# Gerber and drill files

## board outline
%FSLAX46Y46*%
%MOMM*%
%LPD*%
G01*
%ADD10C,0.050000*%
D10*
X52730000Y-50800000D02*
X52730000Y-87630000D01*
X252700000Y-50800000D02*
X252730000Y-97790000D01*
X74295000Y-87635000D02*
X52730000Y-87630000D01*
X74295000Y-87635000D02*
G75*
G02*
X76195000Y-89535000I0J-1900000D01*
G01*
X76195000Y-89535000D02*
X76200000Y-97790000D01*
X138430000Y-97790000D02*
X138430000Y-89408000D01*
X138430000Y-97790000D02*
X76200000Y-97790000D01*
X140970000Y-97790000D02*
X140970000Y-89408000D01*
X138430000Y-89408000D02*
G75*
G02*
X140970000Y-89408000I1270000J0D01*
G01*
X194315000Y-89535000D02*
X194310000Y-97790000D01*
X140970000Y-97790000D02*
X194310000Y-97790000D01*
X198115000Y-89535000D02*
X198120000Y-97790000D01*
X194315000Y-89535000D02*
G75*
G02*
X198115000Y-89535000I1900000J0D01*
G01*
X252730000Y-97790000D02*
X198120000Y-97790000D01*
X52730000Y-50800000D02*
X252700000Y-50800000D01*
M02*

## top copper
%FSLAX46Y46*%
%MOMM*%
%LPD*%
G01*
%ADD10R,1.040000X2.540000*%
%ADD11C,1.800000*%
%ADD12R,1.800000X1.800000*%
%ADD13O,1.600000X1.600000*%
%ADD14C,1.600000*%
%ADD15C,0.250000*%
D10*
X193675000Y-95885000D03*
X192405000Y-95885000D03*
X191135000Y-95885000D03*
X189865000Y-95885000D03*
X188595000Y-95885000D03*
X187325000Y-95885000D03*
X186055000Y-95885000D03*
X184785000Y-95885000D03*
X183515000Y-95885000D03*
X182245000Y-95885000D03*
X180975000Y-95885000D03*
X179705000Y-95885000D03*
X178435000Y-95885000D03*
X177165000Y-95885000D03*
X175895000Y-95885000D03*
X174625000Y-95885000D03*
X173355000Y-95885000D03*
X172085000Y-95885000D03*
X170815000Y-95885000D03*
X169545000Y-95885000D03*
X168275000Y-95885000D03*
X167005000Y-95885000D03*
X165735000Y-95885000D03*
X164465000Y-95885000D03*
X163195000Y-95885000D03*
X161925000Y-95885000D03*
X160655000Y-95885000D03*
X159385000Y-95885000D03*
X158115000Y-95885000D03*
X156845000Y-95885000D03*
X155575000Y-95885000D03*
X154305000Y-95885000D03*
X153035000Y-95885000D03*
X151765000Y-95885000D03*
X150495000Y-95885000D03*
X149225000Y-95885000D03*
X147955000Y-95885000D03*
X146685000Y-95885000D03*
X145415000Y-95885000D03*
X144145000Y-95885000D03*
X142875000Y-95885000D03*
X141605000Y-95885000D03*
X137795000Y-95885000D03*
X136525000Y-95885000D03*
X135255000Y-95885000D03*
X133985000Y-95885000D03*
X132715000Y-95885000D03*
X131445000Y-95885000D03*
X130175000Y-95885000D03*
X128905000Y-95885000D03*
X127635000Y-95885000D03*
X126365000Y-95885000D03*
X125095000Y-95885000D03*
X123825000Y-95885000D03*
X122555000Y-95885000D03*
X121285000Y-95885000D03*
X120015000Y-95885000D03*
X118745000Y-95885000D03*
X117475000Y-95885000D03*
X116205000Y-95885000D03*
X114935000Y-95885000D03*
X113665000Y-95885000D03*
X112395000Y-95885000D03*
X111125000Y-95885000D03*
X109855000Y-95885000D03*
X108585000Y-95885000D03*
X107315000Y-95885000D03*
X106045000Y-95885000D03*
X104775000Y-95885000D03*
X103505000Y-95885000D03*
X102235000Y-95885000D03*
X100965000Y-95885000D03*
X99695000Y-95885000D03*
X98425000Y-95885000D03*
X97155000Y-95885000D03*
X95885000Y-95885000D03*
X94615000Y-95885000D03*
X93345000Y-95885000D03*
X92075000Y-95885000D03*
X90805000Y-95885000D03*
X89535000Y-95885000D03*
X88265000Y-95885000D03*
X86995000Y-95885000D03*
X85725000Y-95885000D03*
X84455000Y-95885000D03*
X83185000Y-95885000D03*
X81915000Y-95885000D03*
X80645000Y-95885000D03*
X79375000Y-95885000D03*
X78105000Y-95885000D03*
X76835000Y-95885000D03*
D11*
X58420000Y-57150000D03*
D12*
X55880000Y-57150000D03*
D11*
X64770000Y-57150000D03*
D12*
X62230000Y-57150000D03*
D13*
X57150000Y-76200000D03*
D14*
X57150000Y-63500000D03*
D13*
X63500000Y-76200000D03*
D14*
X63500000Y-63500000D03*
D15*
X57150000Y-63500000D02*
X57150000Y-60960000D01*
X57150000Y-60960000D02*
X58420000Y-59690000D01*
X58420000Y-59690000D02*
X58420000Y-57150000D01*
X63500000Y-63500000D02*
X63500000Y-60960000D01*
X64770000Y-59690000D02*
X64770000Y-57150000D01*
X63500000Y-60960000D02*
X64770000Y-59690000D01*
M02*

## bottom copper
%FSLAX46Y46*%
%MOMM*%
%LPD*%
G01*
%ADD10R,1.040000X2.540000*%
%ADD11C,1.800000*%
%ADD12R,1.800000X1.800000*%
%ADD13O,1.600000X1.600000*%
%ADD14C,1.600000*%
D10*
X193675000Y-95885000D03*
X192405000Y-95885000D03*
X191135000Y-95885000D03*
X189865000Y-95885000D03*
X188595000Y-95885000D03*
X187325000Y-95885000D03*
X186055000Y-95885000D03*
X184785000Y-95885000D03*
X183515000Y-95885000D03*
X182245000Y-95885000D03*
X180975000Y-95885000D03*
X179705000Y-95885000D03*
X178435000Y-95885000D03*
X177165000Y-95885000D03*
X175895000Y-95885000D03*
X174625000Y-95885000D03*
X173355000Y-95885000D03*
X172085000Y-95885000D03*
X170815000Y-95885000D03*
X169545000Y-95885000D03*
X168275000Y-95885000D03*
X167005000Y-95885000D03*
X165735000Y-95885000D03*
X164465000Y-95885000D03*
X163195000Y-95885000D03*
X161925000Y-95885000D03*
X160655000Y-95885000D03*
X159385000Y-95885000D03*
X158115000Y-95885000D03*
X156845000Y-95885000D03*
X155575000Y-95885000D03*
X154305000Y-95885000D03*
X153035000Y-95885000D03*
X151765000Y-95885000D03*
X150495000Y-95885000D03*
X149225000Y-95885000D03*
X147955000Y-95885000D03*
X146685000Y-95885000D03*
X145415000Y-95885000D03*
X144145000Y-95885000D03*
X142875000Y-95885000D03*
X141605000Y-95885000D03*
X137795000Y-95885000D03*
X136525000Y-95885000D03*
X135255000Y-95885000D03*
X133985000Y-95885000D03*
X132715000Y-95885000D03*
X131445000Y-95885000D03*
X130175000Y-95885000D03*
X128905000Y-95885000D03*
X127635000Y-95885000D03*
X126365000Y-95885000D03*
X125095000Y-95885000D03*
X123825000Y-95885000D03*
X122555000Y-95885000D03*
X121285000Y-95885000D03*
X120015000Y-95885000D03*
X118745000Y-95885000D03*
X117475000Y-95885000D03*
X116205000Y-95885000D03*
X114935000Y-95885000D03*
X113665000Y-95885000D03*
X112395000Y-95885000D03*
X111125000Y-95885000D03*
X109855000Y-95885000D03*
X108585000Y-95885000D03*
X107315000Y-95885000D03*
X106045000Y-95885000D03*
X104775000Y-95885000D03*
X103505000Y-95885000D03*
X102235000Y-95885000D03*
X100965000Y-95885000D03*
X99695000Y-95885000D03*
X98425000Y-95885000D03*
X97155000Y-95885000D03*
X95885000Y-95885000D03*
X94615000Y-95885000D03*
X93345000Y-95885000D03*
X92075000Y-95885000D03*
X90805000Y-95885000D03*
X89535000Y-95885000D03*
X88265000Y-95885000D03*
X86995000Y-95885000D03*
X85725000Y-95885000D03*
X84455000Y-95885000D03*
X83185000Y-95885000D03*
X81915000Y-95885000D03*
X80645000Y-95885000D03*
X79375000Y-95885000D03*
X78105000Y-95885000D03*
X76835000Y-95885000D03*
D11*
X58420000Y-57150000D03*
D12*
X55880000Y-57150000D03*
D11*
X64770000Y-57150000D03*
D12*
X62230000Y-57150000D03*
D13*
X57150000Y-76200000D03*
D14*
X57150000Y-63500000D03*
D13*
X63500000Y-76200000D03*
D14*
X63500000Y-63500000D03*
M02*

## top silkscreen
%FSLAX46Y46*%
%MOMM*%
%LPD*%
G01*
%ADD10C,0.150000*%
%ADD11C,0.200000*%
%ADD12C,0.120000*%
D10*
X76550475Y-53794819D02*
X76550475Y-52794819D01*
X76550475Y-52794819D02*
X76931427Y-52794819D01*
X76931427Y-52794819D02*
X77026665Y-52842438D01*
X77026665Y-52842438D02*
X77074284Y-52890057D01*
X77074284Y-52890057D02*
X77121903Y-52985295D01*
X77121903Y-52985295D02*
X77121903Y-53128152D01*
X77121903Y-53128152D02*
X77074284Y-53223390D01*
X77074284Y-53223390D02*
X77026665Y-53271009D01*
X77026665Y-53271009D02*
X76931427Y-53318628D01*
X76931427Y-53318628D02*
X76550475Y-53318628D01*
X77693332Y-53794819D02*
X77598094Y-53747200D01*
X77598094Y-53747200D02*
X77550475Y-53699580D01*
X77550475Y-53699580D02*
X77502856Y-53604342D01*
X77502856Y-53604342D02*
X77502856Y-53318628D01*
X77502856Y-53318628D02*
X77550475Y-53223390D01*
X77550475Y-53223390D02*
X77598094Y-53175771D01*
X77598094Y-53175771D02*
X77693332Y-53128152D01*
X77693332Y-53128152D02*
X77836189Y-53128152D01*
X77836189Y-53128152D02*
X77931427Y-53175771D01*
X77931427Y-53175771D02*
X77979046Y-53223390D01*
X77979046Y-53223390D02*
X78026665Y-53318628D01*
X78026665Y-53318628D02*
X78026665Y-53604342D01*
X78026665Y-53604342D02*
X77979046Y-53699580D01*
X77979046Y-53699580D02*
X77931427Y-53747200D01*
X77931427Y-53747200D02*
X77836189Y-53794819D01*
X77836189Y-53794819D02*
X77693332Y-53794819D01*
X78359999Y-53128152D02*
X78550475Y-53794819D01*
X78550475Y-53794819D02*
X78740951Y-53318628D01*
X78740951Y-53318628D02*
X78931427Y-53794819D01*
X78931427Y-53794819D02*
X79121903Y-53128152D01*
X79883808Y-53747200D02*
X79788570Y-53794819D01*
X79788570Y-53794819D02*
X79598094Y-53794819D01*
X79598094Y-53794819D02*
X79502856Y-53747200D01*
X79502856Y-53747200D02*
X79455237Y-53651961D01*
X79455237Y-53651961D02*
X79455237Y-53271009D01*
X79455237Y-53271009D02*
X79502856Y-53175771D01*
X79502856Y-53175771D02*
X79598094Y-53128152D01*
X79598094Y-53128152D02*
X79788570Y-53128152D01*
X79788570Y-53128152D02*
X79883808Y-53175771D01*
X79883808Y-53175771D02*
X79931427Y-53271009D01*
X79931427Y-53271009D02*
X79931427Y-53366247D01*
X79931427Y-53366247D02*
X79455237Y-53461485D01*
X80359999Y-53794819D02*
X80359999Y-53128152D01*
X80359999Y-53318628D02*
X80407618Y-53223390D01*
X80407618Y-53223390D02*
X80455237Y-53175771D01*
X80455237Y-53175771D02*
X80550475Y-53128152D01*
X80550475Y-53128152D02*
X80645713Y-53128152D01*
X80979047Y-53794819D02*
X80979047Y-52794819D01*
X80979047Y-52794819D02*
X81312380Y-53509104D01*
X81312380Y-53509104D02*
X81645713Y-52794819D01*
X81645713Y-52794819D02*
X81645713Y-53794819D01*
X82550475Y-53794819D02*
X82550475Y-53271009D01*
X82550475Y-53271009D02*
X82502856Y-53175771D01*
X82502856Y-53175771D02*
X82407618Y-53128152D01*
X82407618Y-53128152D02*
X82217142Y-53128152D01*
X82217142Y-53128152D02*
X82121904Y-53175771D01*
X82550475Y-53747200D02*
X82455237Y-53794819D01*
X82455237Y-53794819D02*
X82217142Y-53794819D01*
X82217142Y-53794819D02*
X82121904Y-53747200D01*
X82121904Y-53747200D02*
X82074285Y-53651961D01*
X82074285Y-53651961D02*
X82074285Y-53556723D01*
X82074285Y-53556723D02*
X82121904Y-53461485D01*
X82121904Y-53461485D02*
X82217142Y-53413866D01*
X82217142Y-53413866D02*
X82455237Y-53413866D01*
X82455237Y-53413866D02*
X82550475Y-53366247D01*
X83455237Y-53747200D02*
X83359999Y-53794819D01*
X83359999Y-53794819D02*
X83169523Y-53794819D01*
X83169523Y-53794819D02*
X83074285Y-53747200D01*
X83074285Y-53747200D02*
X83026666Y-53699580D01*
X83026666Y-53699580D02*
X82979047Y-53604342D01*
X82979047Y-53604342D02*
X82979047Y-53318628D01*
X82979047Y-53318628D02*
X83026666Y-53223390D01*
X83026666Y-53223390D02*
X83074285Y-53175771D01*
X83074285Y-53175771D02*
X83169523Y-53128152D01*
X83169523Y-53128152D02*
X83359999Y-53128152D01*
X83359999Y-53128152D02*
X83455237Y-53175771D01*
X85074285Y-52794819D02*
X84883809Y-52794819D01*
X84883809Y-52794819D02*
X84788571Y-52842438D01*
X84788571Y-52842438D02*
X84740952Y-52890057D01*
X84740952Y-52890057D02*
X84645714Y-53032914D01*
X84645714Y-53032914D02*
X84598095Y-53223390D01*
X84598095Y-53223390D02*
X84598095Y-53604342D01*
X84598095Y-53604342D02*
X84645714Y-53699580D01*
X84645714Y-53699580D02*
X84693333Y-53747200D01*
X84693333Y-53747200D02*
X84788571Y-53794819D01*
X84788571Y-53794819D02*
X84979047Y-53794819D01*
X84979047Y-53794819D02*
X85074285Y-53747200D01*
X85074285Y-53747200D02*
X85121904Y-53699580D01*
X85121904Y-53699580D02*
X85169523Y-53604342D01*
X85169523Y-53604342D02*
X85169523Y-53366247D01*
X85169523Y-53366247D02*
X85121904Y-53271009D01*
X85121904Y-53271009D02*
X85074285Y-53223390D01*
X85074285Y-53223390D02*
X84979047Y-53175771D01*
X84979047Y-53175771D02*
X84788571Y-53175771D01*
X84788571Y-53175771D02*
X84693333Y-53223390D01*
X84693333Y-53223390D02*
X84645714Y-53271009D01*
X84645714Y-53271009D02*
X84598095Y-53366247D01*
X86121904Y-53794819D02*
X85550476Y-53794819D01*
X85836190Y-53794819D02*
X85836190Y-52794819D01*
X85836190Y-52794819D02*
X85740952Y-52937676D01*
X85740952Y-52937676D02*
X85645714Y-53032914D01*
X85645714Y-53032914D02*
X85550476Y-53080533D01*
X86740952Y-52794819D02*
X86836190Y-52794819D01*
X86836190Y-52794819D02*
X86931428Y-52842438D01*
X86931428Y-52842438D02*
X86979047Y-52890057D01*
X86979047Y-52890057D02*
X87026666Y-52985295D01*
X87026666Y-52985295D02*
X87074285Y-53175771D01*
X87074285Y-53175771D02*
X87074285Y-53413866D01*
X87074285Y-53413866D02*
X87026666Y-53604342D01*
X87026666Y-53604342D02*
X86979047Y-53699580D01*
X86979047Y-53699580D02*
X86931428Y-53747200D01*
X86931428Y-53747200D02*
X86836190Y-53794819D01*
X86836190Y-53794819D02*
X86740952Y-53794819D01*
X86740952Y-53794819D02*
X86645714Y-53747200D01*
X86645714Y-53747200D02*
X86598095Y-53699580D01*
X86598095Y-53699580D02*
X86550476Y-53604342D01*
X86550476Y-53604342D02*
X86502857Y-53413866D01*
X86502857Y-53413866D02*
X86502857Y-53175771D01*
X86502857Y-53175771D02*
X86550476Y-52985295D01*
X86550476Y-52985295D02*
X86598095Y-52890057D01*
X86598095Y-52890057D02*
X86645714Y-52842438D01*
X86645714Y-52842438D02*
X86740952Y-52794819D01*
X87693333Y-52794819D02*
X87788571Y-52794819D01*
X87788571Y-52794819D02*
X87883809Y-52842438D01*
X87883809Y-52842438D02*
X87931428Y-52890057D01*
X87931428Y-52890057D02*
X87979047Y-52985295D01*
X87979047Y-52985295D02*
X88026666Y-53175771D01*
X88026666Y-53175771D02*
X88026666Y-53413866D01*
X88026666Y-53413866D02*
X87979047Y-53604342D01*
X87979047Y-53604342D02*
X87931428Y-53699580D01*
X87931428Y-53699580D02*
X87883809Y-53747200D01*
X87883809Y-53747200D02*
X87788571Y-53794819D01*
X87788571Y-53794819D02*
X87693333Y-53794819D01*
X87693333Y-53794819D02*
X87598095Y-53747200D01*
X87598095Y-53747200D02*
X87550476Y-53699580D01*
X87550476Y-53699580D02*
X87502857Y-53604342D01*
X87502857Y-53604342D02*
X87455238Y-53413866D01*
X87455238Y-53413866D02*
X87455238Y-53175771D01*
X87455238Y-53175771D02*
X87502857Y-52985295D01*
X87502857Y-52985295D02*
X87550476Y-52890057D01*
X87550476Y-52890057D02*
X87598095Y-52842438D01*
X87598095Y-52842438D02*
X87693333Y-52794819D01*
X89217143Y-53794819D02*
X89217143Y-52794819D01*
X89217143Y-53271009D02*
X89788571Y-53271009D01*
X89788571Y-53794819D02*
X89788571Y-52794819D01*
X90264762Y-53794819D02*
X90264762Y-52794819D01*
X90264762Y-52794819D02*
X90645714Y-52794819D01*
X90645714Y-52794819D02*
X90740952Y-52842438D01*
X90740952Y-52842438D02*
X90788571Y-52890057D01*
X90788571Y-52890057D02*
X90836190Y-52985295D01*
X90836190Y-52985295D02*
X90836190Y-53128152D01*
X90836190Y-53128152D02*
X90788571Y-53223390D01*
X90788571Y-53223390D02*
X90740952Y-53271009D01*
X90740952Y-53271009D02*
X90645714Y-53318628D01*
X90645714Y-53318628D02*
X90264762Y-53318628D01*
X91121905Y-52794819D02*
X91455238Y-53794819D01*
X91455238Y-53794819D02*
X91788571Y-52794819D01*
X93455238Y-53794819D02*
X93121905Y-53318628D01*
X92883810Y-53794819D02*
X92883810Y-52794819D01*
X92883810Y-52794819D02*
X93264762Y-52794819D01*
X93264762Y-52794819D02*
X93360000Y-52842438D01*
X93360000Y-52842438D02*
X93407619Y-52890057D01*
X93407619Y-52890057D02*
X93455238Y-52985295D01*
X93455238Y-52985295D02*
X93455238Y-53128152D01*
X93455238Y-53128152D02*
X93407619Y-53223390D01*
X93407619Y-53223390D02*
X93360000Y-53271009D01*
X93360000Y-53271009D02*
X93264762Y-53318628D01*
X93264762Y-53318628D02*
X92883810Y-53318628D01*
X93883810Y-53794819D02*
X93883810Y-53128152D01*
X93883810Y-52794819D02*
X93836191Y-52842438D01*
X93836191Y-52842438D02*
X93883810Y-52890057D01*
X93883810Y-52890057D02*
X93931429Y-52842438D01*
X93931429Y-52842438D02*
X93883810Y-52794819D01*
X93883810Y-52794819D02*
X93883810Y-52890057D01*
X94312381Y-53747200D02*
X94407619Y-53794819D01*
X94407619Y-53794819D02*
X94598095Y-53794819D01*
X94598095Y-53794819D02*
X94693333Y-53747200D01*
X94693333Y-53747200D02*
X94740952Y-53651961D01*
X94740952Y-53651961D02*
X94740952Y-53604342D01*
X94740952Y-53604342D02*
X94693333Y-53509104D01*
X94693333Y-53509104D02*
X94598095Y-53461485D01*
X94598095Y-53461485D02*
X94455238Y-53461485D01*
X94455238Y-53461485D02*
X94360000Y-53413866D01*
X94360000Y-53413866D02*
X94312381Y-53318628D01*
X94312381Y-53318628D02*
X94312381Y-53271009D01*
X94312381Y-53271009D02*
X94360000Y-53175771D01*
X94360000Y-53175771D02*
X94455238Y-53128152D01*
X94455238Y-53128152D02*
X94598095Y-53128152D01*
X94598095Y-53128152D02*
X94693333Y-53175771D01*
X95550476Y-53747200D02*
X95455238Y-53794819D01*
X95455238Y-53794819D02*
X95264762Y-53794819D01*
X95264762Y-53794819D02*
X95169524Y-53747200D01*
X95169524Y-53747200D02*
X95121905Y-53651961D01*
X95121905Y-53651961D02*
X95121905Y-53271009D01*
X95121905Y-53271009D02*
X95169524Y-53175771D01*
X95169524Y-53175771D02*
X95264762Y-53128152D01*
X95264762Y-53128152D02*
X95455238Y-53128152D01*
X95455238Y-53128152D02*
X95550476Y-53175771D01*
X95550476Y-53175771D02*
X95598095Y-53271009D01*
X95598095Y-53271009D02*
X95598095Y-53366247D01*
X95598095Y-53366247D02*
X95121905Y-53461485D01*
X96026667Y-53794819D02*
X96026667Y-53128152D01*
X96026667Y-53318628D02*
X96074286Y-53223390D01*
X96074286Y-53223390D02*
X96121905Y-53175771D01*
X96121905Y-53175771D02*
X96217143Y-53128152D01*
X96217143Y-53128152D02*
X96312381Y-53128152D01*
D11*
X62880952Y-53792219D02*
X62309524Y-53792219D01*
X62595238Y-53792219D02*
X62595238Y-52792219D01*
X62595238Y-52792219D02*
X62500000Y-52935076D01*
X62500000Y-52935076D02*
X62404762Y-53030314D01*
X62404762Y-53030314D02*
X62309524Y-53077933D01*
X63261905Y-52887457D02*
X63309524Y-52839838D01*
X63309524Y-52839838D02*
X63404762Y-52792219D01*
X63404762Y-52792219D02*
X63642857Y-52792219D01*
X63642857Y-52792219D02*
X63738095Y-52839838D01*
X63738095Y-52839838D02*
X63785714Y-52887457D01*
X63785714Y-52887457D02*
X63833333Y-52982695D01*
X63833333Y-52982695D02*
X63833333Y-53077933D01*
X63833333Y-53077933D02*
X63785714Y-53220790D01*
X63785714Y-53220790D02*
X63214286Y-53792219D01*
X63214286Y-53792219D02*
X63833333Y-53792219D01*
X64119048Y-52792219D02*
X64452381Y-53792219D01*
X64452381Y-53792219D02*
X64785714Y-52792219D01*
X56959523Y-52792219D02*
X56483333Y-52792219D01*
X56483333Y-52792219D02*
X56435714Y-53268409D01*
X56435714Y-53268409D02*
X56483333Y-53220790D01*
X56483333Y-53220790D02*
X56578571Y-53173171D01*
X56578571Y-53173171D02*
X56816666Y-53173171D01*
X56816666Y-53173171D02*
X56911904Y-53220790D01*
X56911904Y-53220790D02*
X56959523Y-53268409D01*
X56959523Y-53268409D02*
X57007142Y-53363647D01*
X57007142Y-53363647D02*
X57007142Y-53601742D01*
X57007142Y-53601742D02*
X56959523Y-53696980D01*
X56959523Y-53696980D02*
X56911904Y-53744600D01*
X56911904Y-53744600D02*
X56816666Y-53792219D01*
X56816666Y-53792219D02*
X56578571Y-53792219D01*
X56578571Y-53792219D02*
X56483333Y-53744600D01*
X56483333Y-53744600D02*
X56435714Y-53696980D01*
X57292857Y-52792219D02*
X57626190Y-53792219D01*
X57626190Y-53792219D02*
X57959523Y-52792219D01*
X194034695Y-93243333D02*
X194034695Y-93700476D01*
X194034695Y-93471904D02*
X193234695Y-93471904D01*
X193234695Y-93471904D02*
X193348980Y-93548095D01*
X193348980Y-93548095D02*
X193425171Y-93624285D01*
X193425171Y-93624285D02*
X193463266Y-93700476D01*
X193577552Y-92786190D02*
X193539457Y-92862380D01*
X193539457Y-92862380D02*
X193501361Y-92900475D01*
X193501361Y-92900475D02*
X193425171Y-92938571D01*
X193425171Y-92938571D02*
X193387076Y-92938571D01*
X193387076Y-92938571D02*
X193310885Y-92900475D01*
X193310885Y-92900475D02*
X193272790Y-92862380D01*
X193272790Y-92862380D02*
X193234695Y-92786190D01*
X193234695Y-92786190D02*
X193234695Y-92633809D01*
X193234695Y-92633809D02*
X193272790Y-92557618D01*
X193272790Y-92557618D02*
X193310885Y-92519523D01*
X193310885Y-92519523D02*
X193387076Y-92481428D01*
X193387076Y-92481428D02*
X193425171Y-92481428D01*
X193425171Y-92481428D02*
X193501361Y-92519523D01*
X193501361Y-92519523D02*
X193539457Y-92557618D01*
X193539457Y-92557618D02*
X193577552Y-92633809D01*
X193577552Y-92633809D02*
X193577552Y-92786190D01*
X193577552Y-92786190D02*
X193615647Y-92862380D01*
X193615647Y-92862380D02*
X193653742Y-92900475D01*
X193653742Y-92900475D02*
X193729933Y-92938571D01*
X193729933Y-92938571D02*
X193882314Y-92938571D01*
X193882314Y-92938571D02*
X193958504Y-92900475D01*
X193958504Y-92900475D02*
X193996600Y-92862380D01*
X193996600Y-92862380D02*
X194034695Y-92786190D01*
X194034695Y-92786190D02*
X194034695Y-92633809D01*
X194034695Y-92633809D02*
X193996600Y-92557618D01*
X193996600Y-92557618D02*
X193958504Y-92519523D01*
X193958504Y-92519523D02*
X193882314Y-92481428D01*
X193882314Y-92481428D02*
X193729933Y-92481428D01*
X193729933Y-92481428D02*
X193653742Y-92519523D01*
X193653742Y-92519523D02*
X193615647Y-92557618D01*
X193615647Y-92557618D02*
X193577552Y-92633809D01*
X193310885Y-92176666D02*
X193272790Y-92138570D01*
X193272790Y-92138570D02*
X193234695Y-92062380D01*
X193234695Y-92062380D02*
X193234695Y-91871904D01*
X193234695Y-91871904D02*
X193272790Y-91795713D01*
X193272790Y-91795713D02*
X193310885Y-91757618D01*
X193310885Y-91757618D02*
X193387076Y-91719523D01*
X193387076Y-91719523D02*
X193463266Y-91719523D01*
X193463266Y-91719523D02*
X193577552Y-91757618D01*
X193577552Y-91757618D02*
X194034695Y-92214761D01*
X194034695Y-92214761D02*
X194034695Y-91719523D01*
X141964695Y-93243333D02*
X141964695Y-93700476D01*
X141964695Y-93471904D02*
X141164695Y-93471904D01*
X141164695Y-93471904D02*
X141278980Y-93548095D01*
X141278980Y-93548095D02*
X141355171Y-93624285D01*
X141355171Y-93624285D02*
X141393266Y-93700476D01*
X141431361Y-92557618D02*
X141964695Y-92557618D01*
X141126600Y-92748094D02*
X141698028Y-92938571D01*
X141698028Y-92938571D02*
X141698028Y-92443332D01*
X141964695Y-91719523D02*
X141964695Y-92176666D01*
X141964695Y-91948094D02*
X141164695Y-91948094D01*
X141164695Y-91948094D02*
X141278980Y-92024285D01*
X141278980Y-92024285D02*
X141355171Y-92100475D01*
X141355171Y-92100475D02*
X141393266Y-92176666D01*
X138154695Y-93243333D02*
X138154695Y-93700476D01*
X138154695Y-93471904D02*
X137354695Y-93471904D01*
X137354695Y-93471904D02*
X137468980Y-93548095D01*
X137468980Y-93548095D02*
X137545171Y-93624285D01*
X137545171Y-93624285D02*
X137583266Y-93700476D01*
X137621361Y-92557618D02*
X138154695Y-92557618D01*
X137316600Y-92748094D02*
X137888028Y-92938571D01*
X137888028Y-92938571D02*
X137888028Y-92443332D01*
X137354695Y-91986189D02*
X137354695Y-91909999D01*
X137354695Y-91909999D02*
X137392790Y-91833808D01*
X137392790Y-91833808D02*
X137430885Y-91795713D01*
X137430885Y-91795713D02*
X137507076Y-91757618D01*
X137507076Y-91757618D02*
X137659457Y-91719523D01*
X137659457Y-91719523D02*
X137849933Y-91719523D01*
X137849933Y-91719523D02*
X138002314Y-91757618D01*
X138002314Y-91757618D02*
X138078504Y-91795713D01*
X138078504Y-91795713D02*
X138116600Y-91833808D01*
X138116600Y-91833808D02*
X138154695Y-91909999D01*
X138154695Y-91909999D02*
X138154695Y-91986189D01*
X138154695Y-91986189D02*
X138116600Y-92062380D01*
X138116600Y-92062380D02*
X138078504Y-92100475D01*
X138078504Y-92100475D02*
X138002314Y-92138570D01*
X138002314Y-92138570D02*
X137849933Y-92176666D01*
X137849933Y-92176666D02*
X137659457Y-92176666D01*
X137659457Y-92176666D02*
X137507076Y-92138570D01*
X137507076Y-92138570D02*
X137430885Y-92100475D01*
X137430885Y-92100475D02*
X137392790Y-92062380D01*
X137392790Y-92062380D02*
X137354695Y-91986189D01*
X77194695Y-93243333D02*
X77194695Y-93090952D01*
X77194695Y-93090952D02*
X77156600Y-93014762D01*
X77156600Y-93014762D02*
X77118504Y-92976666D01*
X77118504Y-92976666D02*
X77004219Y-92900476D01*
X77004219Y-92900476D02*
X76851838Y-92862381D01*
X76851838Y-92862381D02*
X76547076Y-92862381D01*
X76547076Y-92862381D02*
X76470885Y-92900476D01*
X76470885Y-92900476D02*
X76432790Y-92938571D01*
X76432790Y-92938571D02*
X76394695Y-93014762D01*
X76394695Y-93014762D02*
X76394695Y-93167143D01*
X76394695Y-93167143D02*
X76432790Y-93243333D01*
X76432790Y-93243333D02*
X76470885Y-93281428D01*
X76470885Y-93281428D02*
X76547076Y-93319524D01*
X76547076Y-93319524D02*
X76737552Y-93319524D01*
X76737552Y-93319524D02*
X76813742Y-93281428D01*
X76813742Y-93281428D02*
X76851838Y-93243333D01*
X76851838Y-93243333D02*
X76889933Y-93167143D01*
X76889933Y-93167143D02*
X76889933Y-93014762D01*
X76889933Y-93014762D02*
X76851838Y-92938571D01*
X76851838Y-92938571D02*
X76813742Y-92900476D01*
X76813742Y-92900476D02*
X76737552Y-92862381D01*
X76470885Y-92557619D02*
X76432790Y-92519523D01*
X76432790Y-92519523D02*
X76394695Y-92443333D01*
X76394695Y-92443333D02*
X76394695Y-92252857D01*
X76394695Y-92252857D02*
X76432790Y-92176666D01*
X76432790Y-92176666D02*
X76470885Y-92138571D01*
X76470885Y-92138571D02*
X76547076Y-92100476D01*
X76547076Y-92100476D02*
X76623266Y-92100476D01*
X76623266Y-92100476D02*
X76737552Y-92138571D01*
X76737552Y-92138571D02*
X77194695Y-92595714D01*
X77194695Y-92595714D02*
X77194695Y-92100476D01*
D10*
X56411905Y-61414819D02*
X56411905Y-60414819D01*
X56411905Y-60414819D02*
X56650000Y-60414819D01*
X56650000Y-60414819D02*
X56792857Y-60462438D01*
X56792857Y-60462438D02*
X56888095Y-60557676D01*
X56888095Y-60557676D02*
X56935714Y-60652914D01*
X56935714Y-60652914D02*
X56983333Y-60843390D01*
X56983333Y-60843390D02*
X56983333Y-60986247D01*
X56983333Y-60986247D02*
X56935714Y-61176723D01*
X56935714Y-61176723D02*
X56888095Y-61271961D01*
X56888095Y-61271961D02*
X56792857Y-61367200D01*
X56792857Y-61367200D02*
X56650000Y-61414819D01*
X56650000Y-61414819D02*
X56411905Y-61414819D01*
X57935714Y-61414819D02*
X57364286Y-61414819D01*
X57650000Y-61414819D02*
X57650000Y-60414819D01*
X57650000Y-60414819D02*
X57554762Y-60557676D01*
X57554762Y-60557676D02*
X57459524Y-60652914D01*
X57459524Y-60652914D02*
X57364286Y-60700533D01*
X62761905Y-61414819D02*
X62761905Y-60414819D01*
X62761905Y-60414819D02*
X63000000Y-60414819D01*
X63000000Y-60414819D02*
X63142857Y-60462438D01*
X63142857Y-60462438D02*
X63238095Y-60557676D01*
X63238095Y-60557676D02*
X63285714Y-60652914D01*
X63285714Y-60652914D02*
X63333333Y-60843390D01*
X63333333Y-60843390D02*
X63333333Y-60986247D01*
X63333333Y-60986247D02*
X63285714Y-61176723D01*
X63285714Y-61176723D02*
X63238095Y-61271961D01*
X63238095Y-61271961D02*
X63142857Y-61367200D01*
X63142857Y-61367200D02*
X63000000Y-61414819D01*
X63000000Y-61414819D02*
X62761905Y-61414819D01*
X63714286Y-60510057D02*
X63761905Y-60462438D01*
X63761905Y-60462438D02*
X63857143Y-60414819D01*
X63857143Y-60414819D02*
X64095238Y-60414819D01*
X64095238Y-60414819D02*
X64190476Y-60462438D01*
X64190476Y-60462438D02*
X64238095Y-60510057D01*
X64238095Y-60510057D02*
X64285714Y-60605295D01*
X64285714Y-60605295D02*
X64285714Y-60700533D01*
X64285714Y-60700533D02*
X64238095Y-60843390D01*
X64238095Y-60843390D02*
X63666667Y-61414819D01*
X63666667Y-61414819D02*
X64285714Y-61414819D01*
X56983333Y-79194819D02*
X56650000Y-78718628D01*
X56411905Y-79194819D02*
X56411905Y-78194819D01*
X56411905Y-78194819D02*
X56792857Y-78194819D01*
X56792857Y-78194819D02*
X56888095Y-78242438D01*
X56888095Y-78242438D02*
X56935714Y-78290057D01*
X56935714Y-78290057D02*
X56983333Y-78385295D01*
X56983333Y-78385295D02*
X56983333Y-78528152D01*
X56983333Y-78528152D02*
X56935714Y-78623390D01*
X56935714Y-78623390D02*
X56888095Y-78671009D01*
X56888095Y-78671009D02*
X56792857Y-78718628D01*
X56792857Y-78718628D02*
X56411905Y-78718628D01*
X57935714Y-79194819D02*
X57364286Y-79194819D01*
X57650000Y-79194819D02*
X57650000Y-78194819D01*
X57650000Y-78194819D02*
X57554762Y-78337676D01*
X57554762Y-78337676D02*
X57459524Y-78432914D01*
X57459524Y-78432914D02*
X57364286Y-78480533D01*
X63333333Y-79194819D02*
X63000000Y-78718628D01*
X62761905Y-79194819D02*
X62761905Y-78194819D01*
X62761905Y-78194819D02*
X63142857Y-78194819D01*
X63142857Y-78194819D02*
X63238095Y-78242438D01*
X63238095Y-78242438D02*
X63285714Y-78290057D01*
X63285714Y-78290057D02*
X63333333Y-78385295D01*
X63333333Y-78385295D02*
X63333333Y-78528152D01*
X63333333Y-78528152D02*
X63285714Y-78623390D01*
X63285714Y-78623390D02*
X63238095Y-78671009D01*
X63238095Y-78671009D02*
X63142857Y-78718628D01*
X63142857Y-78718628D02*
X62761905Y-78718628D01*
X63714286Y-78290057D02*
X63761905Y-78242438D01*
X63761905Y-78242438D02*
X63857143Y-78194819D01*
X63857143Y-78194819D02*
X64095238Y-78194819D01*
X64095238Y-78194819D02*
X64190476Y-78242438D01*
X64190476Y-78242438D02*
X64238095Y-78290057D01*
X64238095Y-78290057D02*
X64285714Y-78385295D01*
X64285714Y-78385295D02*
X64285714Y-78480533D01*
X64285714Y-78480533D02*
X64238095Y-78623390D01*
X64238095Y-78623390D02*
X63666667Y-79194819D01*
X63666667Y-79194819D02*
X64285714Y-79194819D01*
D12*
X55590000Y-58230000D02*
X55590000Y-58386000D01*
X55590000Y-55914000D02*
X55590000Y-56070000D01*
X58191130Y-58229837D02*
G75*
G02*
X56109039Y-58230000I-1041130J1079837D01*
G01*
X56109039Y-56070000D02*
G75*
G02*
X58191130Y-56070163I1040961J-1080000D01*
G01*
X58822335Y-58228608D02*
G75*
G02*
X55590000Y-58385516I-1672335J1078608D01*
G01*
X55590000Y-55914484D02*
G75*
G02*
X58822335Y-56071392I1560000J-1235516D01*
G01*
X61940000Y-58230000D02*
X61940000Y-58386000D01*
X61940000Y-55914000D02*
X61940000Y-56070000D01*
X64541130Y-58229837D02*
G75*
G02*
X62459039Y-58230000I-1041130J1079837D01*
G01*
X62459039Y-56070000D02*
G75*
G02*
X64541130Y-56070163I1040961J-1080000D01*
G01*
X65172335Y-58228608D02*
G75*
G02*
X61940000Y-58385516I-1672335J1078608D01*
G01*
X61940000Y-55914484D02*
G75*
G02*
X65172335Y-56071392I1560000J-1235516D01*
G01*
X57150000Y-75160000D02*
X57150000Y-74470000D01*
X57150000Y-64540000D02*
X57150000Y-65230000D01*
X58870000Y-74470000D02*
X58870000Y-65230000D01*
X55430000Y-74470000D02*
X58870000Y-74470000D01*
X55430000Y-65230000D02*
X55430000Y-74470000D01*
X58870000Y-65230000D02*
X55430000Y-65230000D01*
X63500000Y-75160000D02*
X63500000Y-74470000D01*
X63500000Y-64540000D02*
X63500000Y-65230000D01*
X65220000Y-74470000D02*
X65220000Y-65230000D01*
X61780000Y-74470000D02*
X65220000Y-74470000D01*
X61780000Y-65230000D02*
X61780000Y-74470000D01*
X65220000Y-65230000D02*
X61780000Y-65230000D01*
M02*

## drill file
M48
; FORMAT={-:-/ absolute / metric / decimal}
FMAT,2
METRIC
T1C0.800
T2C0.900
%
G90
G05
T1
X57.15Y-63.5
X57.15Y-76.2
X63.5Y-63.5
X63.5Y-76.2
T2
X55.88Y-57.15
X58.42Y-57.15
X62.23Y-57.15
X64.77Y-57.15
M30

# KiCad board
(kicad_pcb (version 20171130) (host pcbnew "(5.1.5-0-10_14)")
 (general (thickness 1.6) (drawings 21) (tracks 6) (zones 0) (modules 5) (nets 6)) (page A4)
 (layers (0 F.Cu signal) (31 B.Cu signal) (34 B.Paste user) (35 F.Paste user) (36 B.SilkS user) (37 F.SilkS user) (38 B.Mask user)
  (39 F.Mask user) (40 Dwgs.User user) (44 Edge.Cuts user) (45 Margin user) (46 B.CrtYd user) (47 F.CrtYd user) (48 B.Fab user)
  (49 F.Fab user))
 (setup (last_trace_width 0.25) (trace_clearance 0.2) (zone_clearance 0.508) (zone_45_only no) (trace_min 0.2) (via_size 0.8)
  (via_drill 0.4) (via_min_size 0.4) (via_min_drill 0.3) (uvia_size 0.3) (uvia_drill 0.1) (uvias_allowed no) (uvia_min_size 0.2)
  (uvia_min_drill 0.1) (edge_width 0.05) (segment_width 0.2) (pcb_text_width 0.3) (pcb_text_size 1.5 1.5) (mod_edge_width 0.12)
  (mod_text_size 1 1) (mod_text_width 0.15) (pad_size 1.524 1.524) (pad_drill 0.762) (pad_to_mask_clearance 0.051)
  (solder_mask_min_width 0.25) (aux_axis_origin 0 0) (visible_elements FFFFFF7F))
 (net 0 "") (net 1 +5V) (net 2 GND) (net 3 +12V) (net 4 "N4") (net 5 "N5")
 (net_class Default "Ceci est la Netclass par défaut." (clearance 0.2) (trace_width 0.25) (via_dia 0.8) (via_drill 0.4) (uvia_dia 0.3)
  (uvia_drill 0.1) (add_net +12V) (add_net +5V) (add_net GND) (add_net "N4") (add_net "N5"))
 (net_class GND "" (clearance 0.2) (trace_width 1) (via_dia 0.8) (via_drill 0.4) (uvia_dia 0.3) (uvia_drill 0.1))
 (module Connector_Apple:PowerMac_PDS (layer F.Cu) (at 135.255 95.885)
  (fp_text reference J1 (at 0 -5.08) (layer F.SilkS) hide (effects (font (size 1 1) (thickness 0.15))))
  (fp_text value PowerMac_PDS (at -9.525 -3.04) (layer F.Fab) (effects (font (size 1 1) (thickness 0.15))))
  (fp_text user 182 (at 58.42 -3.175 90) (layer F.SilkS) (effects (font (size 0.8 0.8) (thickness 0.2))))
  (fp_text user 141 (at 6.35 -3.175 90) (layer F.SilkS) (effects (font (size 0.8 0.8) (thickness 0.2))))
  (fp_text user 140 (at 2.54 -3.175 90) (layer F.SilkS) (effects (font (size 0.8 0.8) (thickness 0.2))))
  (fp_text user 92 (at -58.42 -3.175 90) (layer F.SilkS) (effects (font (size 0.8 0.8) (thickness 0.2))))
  (pad 91 connect rect (at 58.42 0) (size 1.04 2.54) (layers B.Cu B.Mask) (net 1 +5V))
  (pad 90 connect rect (at 57.15 0) (size 1.04 2.54) (layers B.Cu B.Mask) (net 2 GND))
  (pad 89 connect rect (at 55.88 0) (size 1.04 2.54) (layers B.Cu B.Mask))
  (pad 88 connect rect (at 54.61 0) (size 1.04 2.54) (layers B.Cu B.Mask) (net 2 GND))
  (pad 87 connect rect (at 53.34 0) (size 1.04 2.54) (layers B.Cu B.Mask))
  (pad 86 connect rect (at 52.07 0) (size 1.04 2.54) (layers B.Cu B.Mask) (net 1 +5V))
  (pad 85 connect rect (at 50.8 0) (size 1.04 2.54) (layers B.Cu B.Mask) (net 2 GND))
  (pad 84 connect rect (at 49.53 0) (size 1.04 2.54) (layers B.Cu B.Mask))
  (pad 83 connect rect (at 48.26 0) (size 1.04 2.54) (layers B.Cu B.Mask))
  (pad 82 connect rect (at 46.99 0) (size 1.04 2.54) (layers B.Cu B.Mask))
  (pad 81 connect rect (at 45.72 0) (size 1.04 2.54) (layers B.Cu B.Mask))
  (pad 80 connect rect (at 44.45 0) (size 1.04 2.54) (layers B.Cu B.Mask) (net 2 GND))
  (pad 79 connect rect (at 43.18 0) (size 1.04 2.54) (layers B.Cu B.Mask))
  (pad 78 connect rect (at 41.91 0) (size 1.04 2.54) (layers B.Cu B.Mask))
  (pad 77 connect rect (at 40.64 0) (size 1.04 2.54) (layers B.Cu B.Mask))
  (pad 76 connect rect (at 39.37 0) (size 1.04 2.54) (layers B.Cu B.Mask))
  (pad 75 connect rect (at 38.1 0) (size 1.04 2.54) (layers B.Cu B.Mask) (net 1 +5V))
  (pad 74 connect rect (at 36.83 0) (size 1.04 2.54) (layers B.Cu B.Mask))
  (pad 73 connect rect (at 35.56 0) (size 1.04 2.54) (layers B.Cu B.Mask))
  (pad 72 connect rect (at 34.29 0) (size 1.04 2.54) (layers B.Cu B.Mask))
  (pad 71 connect rect (at 33.02 0) (size 1.04 2.54) (layers B.Cu B.Mask))
  (pad 70 connect rect (at 31.75 0) (size 1.04 2.54) (layers B.Cu B.Mask))
  (pad 69 connect rect (at 30.48 0) (size 1.04 2.54) (layers B.Cu B.Mask) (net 2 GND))
  (pad 68 connect rect (at 29.21 0) (size 1.04 2.54) (layers B.Cu B.Mask))
  (pad 67 connect rect (at 27.94 0) (size 1.04 2.54) (layers B.Cu B.Mask))
  (pad 66 connect rect (at 26.67 0) (size 1.04 2.54) (layers B.Cu B.Mask))
  (pad 65 connect rect (at 25.4 0) (size 1.04 2.54) (layers B.Cu B.Mask))
  (pad 64 connect rect (at 24.13 0) (size 1.04 2.54) (layers B.Cu B.Mask) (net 2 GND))
  (pad 63 connect rect (at 22.86 0) (size 1.04 2.54) (layers B.Cu B.Mask))
  (pad 62 connect rect (at 21.59 0) (size 1.04 2.54) (layers B.Cu B.Mask))
  (pad 61 connect rect (at 20.32 0) (size 1.04 2.54) (layers B.Cu B.Mask))
  (pad 60 connect rect (at 19.05 0) (size 1.04 2.54) (layers B.Cu B.Mask))
  (pad 59 connect rect (at 17.78 0) (size 1.04 2.54) (layers B.Cu B.Mask) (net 1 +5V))
  (pad 58 connect rect (at 16.51 0) (size 1.04 2.54) (layers B.Cu B.Mask))
  (pad 57 connect rect (at 15.24 0) (size 1.04 2.54) (layers B.Cu B.Mask))
  (pad 56 connect rect (at 13.97 0) (size 1.04 2.54) (layers B.Cu B.Mask))
  (pad 55 connect rect (at 12.7 0) (size 1.04 2.54) (layers B.Cu B.Mask))
  (pad 54 connect rect (at 11.43 0) (size 1.04 2.54) (layers B.Cu B.Mask))
  (pad 53 connect rect (at 10.16 0) (size 1.04 2.54) (layers B.Cu B.Mask))
  (pad 52 connect rect (at 8.89 0) (size 1.04 2.54) (layers B.Cu B.Mask))
  (pad 51 connect rect (at 7.62 0) (size 1.04 2.54) (layers B.Cu B.Mask))
  (pad 50 connect rect (at 6.35 0) (size 1.04 2.54) (layers B.Cu B.Mask) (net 2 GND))
  (pad 49 connect rect (at 2.54 0) (size 1.04 2.54) (layers B.Cu B.Mask))
  (pad 48 connect rect (at 1.27 0) (size 1.04 2.54) (layers B.Cu B.Mask))
  (pad 47 connect rect (at 0 0) (size 1.04 2.54) (layers B.Cu B.Mask))
  (pad 46 connect rect (at -1.27 0) (size 1.04 2.54) (layers B.Cu B.Mask))
  (pad 45 connect rect (at -2.54 0) (size 1.04 2.54) (layers B.Cu B.Mask) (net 1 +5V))
  (pad 44 connect rect (at -3.81 0) (size 1.04 2.54) (layers B.Cu B.Mask))
  (pad 43 connect rect (at -5.08 0) (size 1.04 2.54) (layers B.Cu B.Mask))
  (pad 42 connect rect (at -6.35 0) (size 1.04 2.54) (layers B.Cu B.Mask))
  (pad 41 connect rect (at -7.62 0) (size 1.04 2.54) (layers B.Cu B.Mask))
  (pad 40 connect rect (at -8.89 0) (size 1.04 2.54) (layers B.Cu B.Mask))
  (pad 39 connect rect (at -10.16 0) (size 1.04 2.54) (layers B.Cu B.Mask) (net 2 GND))
  (pad 38 connect rect (at -11.43 0) (size 1.04 2.54) (layers B.Cu B.Mask))
  (pad 37 connect rect (at -12.7 0) (size 1.04 2.54) (layers B.Cu B.Mask))
  (pad 36 connect rect (at -13.97 0) (size 1.04 2.54) (layers B.Cu B.Mask))
  (pad 35 connect rect (at -15.24 0) (size 1.04 2.54) (layers B.Cu B.Mask))
  (pad 34 connect rect (at -16.51 0) (size 1.04 2.54) (layers B.Cu B.Mask))
  (pad 33 connect rect (at -17.78 0) (size 1.04 2.54) (layers B.Cu B.Mask))
  (pad 32 connect rect (at -19.05 0) (size 1.04 2.54) (layers B.Cu B.Mask) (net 1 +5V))
  (pad 31 connect rect (at -20.32 0) (size 1.04 2.54) (layers B.Cu B.Mask))
  (pad 30 connect rect (at -21.59 0) (size 1.04 2.54) (layers B.Cu B.Mask))
  (pad 29 connect rect (at -22.86 0) (size 1.04 2.54) (layers B.Cu B.Mask))
  (pad 28 connect rect (at -24.13 0) (size 1.04 2.54) (layers B.Cu B.Mask))
  (pad 27 connect rect (at -25.4 0) (size 1.04 2.54) (layers B.Cu B.Mask) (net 2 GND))
  (pad 26 connect rect (at -26.67 0) (size 1.04 2.54) (layers B.Cu B.Mask))
  (pad 25 connect rect (at -27.94 0) (size 1.04 2.54) (layers B.Cu B.Mask))
  (pad 24 connect rect (at -29.21 0) (size 1.04 2.54) (layers B.Cu B.Mask))
  (pad 23 connect rect (at -30.48 0) (size 1.04 2.54) (layers B.Cu B.Mask))
  (pad 22 connect rect (at -31.75 0) (size 1.04 2.54) (layers B.Cu B.Mask) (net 2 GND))
  (pad 21 connect rect (at -33.02 0) (size 1.04 2.54) (layers B.Cu B.Mask))
  (pad 20 connect rect (at -34.29 0) (size 1.04 2.54) (layers B.Cu B.Mask))
  (pad 19 connect rect (at -35.56 0) (size 1.04 2.54) (layers B.Cu B.Mask))
  (pad 18 connect rect (at -36.83 0) (size 1.04 2.54) (layers B.Cu B.Mask))
  (pad 17 connect rect (at -38.1 0) (size 1.04 2.54) (layers B.Cu B.Mask))
  (pad 16 connect rect (at -39.37 0) (size 1.04 2.54) (layers B.Cu B.Mask) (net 1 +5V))
  (pad 15 connect rect (at -40.64 0) (size 1.04 2.54) (layers B.Cu B.Mask))
  (pad 14 connect rect (at -41.91 0) (size 1.04 2.54) (layers B.Cu B.Mask))
  (pad 13 connect rect (at -43.18 0) (size 1.04 2.54) (layers B.Cu B.Mask))
  (pad 12 connect rect (at -44.45 0) (size 1.04 2.54) (layers B.Cu B.Mask))
  (pad 11 connect rect (at -45.72 0) (size 1.04 2.54) (layers B.Cu B.Mask) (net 2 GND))
  (pad 10 connect rect (at -46.99 0) (size 1.04 2.54) (layers B.Cu B.Mask))
  (pad 9 connect rect (at -48.26 0) (size 1.04 2.54) (layers B.Cu B.Mask))
  (pad 8 connect rect (at -49.53 0) (size 1.04 2.54) (layers B.Cu B.Mask))
  (pad 7 connect rect (at -50.8 0) (size 1.04 2.54) (layers B.Cu B.Mask))
  (pad 6 connect rect (at -52.07 0) (size 1.04 2.54) (layers B.Cu B.Mask) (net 2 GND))
  (pad 5 connect rect (at -53.34 0) (size 1.04 2.54) (layers B.Cu B.Mask))
  (pad 4 connect rect (at -54.61 0) (size 1.04 2.54) (layers B.Cu B.Mask))
  (pad 3 connect rect (at -55.88 0) (size 1.04 2.54) (layers B.Cu B.Mask))
  (pad 2 connect rect (at -57.15 0) (size 1.04 2.54) (layers B.Cu B.Mask) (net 2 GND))
  (pad 1 connect rect (at -58.42 0) (size 1.04 2.54) (layers B.Cu B.Mask) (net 1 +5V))
  (pad 182 connect rect (at 58.42 0) (size 1.04 2.54) (layers F.Cu F.Mask) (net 1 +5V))
  (pad 181 connect rect (at 57.15 0) (size 1.04 2.54) (layers F.Cu F.Mask) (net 2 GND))
  (pad 180 connect rect (at 55.88 0) (size 1.04 2.54) (layers F.Cu F.Mask))
  (pad 179 connect rect (at 54.61 0) (size 1.04 2.54) (layers F.Cu F.Mask))
  (pad 178 connect rect (at 53.34 0) (size 1.04 2.54) (layers F.Cu F.Mask))
  (pad 177 connect rect (at 52.07 0) (size 1.04 2.54) (layers F.Cu F.Mask) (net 1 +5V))
  (pad 176 connect rect (at 50.8 0) (size 1.04 2.54) (layers F.Cu F.Mask) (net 2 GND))
  (pad 175 connect rect (at 49.53 0) (size 1.04 2.54) (layers F.Cu F.Mask))
  (pad 174 connect rect (at 48.26 0) (size 1.04 2.54) (layers F.Cu F.Mask))
  (pad 173 connect rect (at 46.99 0) (size 1.04 2.54) (layers F.Cu F.Mask))
  (pad 172 connect rect (at 45.72 0) (size 1.04 2.54) (layers F.Cu F.Mask))
  (pad 171 connect rect (at 44.45 0) (size 1.04 2.54) (layers F.Cu F.Mask) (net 2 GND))
  (pad 170 connect rect (at 43.18 0) (size 1.04 2.54) (layers F.Cu F.Mask))
  (pad 169 connect rect (at 41.91 0) (size 1.04 2.54) (layers F.Cu F.Mask))
  (pad 168 connect rect (at 40.64 0) (size 1.04 2.54) (layers F.Cu F.Mask))
  (pad 167 connect rect (at 39.37 0) (size 1.04 2.54) (layers F.Cu F.Mask))
  (pad 166 connect rect (at 38.1 0) (size 1.04 2.54) (layers F.Cu F.Mask) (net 1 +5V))
  (pad 165 connect rect (at 36.83 0) (size 1.04 2.54) (layers F.Cu F.Mask))
  (pad 164 connect rect (at 35.56 0) (size 1.04 2.54) (layers F.Cu F.Mask))
  (pad 163 connect rect (at 34.29 0) (size 1.04 2.54) (layers F.Cu F.Mask))
  (pad 162 connect rect (at 33.02 0) (size 1.04 2.54) (layers F.Cu F.Mask))
  (pad 161 connect rect (at 31.75 0) (size 1.04 2.54) (layers F.Cu F.Mask))
  (pad 160 connect rect (at 30.48 0) (size 1.04 2.54) (layers F.Cu F.Mask) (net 2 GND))
  (pad 159 connect rect (at 29.21 0) (size 1.04 2.54) (layers F.Cu F.Mask))
  (pad 158 connect rect (at 27.94 0) (size 1.04 2.54) (layers F.Cu F.Mask))
  (pad 157 connect rect (at 26.67 0) (size 1.04 2.54) (layers F.Cu F.Mask))
  (pad 156 connect rect (at 25.4 0) (size 1.04 2.54) (layers F.Cu F.Mask))
  (pad 155 connect rect (at 24.13 0) (size 1.04 2.54) (layers F.Cu F.Mask) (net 2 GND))
  (pad 154 connect rect (at 22.86 0) (size 1.04 2.54) (layers F.Cu F.Mask))
  (pad 153 connect rect (at 21.59 0) (size 1.04 2.54) (layers F.Cu F.Mask))
  (pad 152 connect rect (at 20.32 0) (size 1.04 2.54) (layers F.Cu F.Mask))
  (pad 151 connect rect (at 19.05 0) (size 1.04 2.54) (layers F.Cu F.Mask))
  (pad 150 connect rect (at 17.78 0) (size 1.04 2.54) (layers F.Cu F.Mask) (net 1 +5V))
  (pad 149 connect rect (at 16.51 0) (size 1.04 2.54) (layers F.Cu F.Mask))
  (pad 148 connect rect (at 15.24 0) (size 1.04 2.54) (layers F.Cu F.Mask))
  (pad 147 connect rect (at 13.97 0) (size 1.04 2.54) (layers F.Cu F.Mask))
  (pad 146 connect rect (at 12.7 0) (size 1.04 2.54) (layers F.Cu F.Mask))
  (pad 145 connect rect (at 11.43 0) (size 1.04 2.54) (layers F.Cu F.Mask))
  (pad 144 connect rect (at 10.16 0) (size 1.04 2.54) (layers F.Cu F.Mask))
  (pad 143 connect rect (at 8.89 0) (size 1.04 2.54) (layers F.Cu F.Mask))
  (pad 142 connect rect (at 7.62 0) (size 1.04 2.54) (layers F.Cu F.Mask))
  (pad 141 connect rect (at 6.35 0) (size 1.04 2.54) (layers F.Cu F.Mask) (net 2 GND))
  (pad 140 connect rect (at 2.54 0) (size 1.04 2.54) (layers F.Cu F.Mask))
  (pad 139 connect rect (at 1.27 0) (size 1.04 2.54) (layers F.Cu F.Mask))
  (pad 138 connect rect (at 0 0) (size 1.04 2.54) (layers F.Cu F.Mask))
  (pad 137 connect rect (at -1.27 0) (size 1.04 2.54) (layers F.Cu F.Mask))
  (pad 136 connect rect (at -2.54 0) (size 1.04 2.54) (layers F.Cu F.Mask) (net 1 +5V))
  (pad 135 connect rect (at -3.81 0) (size 1.04 2.54) (layers F.Cu F.Mask))
  (pad 134 connect rect (at -5.08 0) (size 1.04 2.54) (layers F.Cu F.Mask))
  (pad 133 connect rect (at -6.35 0) (size 1.04 2.54) (layers F.Cu F.Mask))
  (pad 132 connect rect (at -7.62 0) (size 1.04 2.54) (layers F.Cu F.Mask))
  (pad 131 connect rect (at -8.89 0) (size 1.04 2.54) (layers F.Cu F.Mask))
  (pad 130 connect rect (at -10.16 0) (size 1.04 2.54) (layers F.Cu F.Mask) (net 2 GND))
  (pad 129 connect rect (at -11.43 0) (size 1.04 2.54) (layers F.Cu F.Mask))
  (pad 128 connect rect (at -12.7 0) (size 1.04 2.54) (layers F.Cu F.Mask))
  (pad 127 connect rect (at -13.97 0) (size 1.04 2.54) (layers F.Cu F.Mask))
  (pad 126 connect rect (at -15.24 0) (size 1.04 2.54) (layers F.Cu F.Mask))
  (pad 125 connect rect (at -16.51 0) (size 1.04 2.54) (layers F.Cu F.Mask))
  (pad 124 connect rect (at -17.78 0) (size 1.04 2.54) (layers F.Cu F.Mask))
  (pad 123 connect rect (at -19.05 0) (size 1.04 2.54) (layers F.Cu F.Mask) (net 1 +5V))
  (pad 122 connect rect (at -20.32 0) (size 1.04 2.54) (layers F.Cu F.Mask))
  (pad 121 connect rect (at -21.59 0) (size 1.04 2.54) (layers F.Cu F.Mask))
  (pad 120 connect rect (at -22.86 0) (size 1.04 2.54) (layers F.Cu F.Mask))
  (pad 119 connect rect (at -24.13 0) (size 1.04 2.54) (layers F.Cu F.Mask))
  (pad 118 connect rect (at -25.4 0) (size 1.04 2.54) (layers F.Cu F.Mask) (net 2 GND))
  (pad 117 connect rect (at -26.67 0) (size 1.04 2.54) (layers F.Cu F.Mask))
  (pad 116 connect rect (at -27.94 0) (size 1.04 2.54) (layers F.Cu F.Mask))
  (pad 115 connect rect (at -29.21 0) (size 1.04 2.54) (layers F.Cu F.Mask))
  (pad 114 connect rect (at -30.48 0) (size 1.04 2.54) (layers F.Cu F.Mask))
  (pad 113 connect rect (at -31.75 0) (size 1.04 2.54) (layers F.Cu F.Mask) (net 2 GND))
  (pad 112 connect rect (at -33.02 0) (size 1.04 2.54) (layers F.Cu F.Mask))
  (pad 111 connect rect (at -34.29 0) (size 1.04 2.54) (layers F.Cu F.Mask))
  (pad 110 connect rect (at -35.56 0) (size 1.04 2.54) (layers F.Cu F.Mask))
  (pad 109 connect rect (at -36.83 0) (size 1.04 2.54) (layers F.Cu F.Mask))
  (pad 108 connect rect (at -38.1 0) (size 1.04 2.54) (layers F.Cu F.Mask))
  (pad 107 connect rect (at -39.37 0) (size 1.04 2.54) (layers F.Cu F.Mask) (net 1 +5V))
  (pad 106 connect rect (at -40.64 0) (size 1.04 2.54) (layers F.Cu F.Mask))
  (pad 105 connect rect (at -41.91 0) (size 1.04 2.54) (layers F.Cu F.Mask))
  (pad 104 connect rect (at -43.18 0) (size 1.04 2.54) (layers F.Cu F.Mask))
  (pad 103 connect rect (at -44.45 0) (size 1.04 2.54) (layers F.Cu F.Mask))
  (pad 102 connect rect (at -45.72 0) (size 1.04 2.54) (layers F.Cu F.Mask) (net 2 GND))
  (pad 101 connect rect (at -46.99 0) (size 1.04 2.54) (layers F.Cu F.Mask))
  (pad 100 connect rect (at -48.26 0) (size 1.04 2.54) (layers F.Cu F.Mask))
  (pad 99 connect rect (at -49.53 0) (size 1.04 2.54) (layers F.Cu F.Mask))
  (pad 98 connect rect (at -50.8 0) (size 1.04 2.54) (layers F.Cu F.Mask))
  (pad 97 connect rect (at -52.07 0) (size 1.04 2.54) (layers F.Cu F.Mask) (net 2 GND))
  (pad 96 connect rect (at -53.34 0) (size 1.04 2.54) (layers F.Cu F.Mask))
  (pad 95 connect rect (at -54.61 0) (size 1.04 2.54) (layers F.Cu F.Mask) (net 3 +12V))
  (pad 94 connect rect (at -55.88 0) (size 1.04 2.54) (layers F.Cu F.Mask) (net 3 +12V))
  (pad 93 connect rect (at -57.15 0) (size 1.04 2.54) (layers F.Cu F.Mask) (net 2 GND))
  (pad 92 connect rect (at -58.42 0) (size 1.04 2.54) (layers F.Cu F.Mask) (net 1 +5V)))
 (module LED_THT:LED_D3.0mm (layer F.Cu) (at 55.88 57.15)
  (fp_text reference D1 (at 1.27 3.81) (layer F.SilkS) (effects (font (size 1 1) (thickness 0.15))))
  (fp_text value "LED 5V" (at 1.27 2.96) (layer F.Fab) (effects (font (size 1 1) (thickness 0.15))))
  (fp_line (start -0.29 1.08) (end -0.29 1.236) (layer F.SilkS) (width 0.12))
  (fp_line (start -0.29 -1.236) (end -0.29 -1.08) (layer F.SilkS) (width 0.12))
  (fp_arc (start 1.27 0) (end 0.229039 1.08) (angle -87.9) (layer F.SilkS) (width 0.12))
  (fp_arc (start 1.27 0) (end 0.229039 -1.08) (angle 87.9) (layer F.SilkS) (width 0.12))
  (fp_arc (start 1.27 0) (end -0.29 1.235516) (angle -108.8) (layer F.SilkS) (width 0.12))
  (fp_arc (start 1.27 0) (end -0.29 -1.235516) (angle 108.8) (layer F.SilkS) (width 0.12))
  (pad 2 thru_hole circle (at 2.54 0) (size 1.8 1.8) (drill 0.9) (layers *.Cu *.Mask) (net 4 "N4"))
  (pad 1 thru_hole rect (at 0 0) (size 1.8 1.8) (drill 0.9) (layers *.Cu *.Mask) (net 2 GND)))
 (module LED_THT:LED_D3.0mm (layer F.Cu) (at 62.23 57.15)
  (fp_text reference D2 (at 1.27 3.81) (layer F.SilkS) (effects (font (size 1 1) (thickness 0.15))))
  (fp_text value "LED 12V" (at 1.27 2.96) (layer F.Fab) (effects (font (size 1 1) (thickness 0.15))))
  (fp_line (start -0.29 1.08) (end -0.29 1.236) (layer F.SilkS) (width 0.12))
  (fp_line (start -0.29 -1.236) (end -0.29 -1.08) (layer F.SilkS) (width 0.12))
  (fp_arc (start 1.27 0) (end 0.229039 1.08) (angle -87.9) (layer F.SilkS) (width 0.12))
  (fp_arc (start 1.27 0) (end 0.229039 -1.08) (angle 87.9) (layer F.SilkS) (width 0.12))
  (fp_arc (start 1.27 0) (end -0.29 1.235516) (angle -108.8) (layer F.SilkS) (width 0.12))
  (fp_arc (start 1.27 0) (end -0.29 -1.235516) (angle 108.8) (layer F.SilkS) (width 0.12))
  (pad 2 thru_hole circle (at 2.54 0) (size 1.8 1.8) (drill 0.9) (layers *.Cu *.Mask) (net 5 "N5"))
  (pad 1 thru_hole rect (at 0 0) (size 1.8 1.8) (drill 0.9) (layers *.Cu *.Mask) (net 2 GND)))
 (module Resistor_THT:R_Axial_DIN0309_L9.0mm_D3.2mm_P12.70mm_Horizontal (layer F.Cu) (at 57.15 63.5 270)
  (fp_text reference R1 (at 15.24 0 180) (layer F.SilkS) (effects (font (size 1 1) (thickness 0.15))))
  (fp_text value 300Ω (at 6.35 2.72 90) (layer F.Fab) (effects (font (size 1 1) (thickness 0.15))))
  (fp_line (start 11.66 0) (end 10.97 0) (layer F.SilkS) (width 0.12))
  (fp_line (start 1.04 0) (end 1.73 0) (layer F.SilkS) (width 0.12))
  (fp_line (start 10.97 -1.72) (end 1.73 -1.72) (layer F.SilkS) (width 0.12))
  (fp_line (start 10.97 1.72) (end 10.97 -1.72) (layer F.SilkS) (width 0.12))
  (fp_line (start 1.73 1.72) (end 10.97 1.72) (layer F.SilkS) (width 0.12))
  (fp_line (start 1.73 -1.72) (end 1.73 1.72) (layer F.SilkS) (width 0.12))
  (pad 2 thru_hole oval (at 12.7 0 270) (size 1.6 1.6) (drill 0.8) (layers *.Cu *.Mask) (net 1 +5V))
  (pad 1 thru_hole circle (at 0 0 270) (size 1.6 1.6) (drill 0.8) (layers *.Cu *.Mask) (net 4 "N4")))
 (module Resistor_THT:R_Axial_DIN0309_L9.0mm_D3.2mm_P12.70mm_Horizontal (layer F.Cu) (at 63.5 63.5 270)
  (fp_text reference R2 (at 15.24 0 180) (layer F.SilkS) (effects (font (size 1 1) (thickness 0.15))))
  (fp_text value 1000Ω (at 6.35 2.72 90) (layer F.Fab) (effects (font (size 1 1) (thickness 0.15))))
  (fp_line (start 11.66 0) (end 10.97 0) (layer F.SilkS) (width 0.12))
  (fp_line (start 1.04 0) (end 1.73 0) (layer F.SilkS) (width 0.12))
  (fp_line (start 10.97 -1.72) (end 1.73 -1.72) (layer F.SilkS) (width 0.12))
  (fp_line (start 10.97 1.72) (end 10.97 -1.72) (layer F.SilkS) (width 0.12))
  (fp_line (start 1.73 1.72) (end 10.97 1.72) (layer F.SilkS) (width 0.12))
  (fp_line (start 1.73 -1.72) (end 1.73 1.72) (layer F.SilkS) (width 0.12))
  (pad 2 thru_hole oval (at 12.7 0 270) (size 1.6 1.6) (drill 0.8) (layers *.Cu *.Mask) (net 3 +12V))
  (pad 1 thru_hole circle (at 0 0 270) (size 1.6 1.6) (drill 0.8) (layers *.Cu *.Mask) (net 5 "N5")))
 (gr_line (start 52.73 50.8) (end 52.73 87.63) (layer Edge.Cuts) (width 0.05))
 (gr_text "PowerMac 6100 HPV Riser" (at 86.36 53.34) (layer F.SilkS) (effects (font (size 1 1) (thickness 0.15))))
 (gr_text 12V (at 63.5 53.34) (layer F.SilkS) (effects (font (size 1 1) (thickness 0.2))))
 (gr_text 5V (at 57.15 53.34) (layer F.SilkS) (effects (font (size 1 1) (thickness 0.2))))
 (gr_line (start 252.7 50.8) (end 252.73 97.79) (layer Edge.Cuts) (width 0.05))
 (gr_line (start 74.295 87.635) (end 52.73 87.63) (layer Edge.Cuts) (width 0.05))
 (gr_arc (start 74.295 89.535) (end 76.195 89.535) (angle -90) (layer Edge.Cuts) (width 0.05))
 (gr_line (start 76.195 89.535) (end 76.2 97.79) (layer Edge.Cuts) (width 0.05))
 (gr_line (start 138.43 97.79) (end 138.43 89.408) (layer Edge.Cuts) (width 0.05))
 (gr_line (start 138.43 97.79) (end 76.2 97.79) (layer Edge.Cuts) (width 0.05))
 (gr_line (start 140.97 97.79) (end 140.97 89.408) (layer Edge.Cuts) (width 0.05))
 (gr_arc (start 139.7 89.408) (end 140.97 89.408) (angle -180) (layer Edge.Cuts) (width 0.05))
 (gr_line (start 194.315 89.535) (end 194.31 97.79) (layer Edge.Cuts) (width 0.05))
 (gr_line (start 140.97 97.79) (end 194.31 97.79) (layer Edge.Cuts) (width 0.05))
 (gr_line (start 198.115 89.535) (end 198.12 97.79) (layer Edge.Cuts) (width 0.05))
 (gr_arc (start 196.215 89.535) (end 198.115 89.535) (angle -180) (layer Edge.Cuts) (width 0.05))
 (gr_line (start 252.73 97.79) (end 198.12 97.79) (layer Edge.Cuts) (width 0.05))
 (gr_line (start 52.73 50.8) (end 252.7 50.8) (layer Edge.Cuts) (width 0.05))
 (segment (start 57.15 63.5) (end 57.15 60.96) (width 0.25) (layer F.Cu) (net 4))
 (segment (start 57.15 60.96) (end 58.42 59.69) (width 0.25) (layer F.Cu) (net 4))
 (segment (start 58.42 59.69) (end 58.42 57.15) (width 0.25) (layer F.Cu) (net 4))
 (segment (start 63.5 63.5) (end 63.5 60.96) (width 0.25) (layer F.Cu) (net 5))
 (segment (start 64.77 59.69) (end 64.77 57.15) (width 0.25) (layer F.Cu) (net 5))
 (segment (start 63.5 60.96) (end 64.77 59.69) (width 0.25) (layer F.Cu) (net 5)))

